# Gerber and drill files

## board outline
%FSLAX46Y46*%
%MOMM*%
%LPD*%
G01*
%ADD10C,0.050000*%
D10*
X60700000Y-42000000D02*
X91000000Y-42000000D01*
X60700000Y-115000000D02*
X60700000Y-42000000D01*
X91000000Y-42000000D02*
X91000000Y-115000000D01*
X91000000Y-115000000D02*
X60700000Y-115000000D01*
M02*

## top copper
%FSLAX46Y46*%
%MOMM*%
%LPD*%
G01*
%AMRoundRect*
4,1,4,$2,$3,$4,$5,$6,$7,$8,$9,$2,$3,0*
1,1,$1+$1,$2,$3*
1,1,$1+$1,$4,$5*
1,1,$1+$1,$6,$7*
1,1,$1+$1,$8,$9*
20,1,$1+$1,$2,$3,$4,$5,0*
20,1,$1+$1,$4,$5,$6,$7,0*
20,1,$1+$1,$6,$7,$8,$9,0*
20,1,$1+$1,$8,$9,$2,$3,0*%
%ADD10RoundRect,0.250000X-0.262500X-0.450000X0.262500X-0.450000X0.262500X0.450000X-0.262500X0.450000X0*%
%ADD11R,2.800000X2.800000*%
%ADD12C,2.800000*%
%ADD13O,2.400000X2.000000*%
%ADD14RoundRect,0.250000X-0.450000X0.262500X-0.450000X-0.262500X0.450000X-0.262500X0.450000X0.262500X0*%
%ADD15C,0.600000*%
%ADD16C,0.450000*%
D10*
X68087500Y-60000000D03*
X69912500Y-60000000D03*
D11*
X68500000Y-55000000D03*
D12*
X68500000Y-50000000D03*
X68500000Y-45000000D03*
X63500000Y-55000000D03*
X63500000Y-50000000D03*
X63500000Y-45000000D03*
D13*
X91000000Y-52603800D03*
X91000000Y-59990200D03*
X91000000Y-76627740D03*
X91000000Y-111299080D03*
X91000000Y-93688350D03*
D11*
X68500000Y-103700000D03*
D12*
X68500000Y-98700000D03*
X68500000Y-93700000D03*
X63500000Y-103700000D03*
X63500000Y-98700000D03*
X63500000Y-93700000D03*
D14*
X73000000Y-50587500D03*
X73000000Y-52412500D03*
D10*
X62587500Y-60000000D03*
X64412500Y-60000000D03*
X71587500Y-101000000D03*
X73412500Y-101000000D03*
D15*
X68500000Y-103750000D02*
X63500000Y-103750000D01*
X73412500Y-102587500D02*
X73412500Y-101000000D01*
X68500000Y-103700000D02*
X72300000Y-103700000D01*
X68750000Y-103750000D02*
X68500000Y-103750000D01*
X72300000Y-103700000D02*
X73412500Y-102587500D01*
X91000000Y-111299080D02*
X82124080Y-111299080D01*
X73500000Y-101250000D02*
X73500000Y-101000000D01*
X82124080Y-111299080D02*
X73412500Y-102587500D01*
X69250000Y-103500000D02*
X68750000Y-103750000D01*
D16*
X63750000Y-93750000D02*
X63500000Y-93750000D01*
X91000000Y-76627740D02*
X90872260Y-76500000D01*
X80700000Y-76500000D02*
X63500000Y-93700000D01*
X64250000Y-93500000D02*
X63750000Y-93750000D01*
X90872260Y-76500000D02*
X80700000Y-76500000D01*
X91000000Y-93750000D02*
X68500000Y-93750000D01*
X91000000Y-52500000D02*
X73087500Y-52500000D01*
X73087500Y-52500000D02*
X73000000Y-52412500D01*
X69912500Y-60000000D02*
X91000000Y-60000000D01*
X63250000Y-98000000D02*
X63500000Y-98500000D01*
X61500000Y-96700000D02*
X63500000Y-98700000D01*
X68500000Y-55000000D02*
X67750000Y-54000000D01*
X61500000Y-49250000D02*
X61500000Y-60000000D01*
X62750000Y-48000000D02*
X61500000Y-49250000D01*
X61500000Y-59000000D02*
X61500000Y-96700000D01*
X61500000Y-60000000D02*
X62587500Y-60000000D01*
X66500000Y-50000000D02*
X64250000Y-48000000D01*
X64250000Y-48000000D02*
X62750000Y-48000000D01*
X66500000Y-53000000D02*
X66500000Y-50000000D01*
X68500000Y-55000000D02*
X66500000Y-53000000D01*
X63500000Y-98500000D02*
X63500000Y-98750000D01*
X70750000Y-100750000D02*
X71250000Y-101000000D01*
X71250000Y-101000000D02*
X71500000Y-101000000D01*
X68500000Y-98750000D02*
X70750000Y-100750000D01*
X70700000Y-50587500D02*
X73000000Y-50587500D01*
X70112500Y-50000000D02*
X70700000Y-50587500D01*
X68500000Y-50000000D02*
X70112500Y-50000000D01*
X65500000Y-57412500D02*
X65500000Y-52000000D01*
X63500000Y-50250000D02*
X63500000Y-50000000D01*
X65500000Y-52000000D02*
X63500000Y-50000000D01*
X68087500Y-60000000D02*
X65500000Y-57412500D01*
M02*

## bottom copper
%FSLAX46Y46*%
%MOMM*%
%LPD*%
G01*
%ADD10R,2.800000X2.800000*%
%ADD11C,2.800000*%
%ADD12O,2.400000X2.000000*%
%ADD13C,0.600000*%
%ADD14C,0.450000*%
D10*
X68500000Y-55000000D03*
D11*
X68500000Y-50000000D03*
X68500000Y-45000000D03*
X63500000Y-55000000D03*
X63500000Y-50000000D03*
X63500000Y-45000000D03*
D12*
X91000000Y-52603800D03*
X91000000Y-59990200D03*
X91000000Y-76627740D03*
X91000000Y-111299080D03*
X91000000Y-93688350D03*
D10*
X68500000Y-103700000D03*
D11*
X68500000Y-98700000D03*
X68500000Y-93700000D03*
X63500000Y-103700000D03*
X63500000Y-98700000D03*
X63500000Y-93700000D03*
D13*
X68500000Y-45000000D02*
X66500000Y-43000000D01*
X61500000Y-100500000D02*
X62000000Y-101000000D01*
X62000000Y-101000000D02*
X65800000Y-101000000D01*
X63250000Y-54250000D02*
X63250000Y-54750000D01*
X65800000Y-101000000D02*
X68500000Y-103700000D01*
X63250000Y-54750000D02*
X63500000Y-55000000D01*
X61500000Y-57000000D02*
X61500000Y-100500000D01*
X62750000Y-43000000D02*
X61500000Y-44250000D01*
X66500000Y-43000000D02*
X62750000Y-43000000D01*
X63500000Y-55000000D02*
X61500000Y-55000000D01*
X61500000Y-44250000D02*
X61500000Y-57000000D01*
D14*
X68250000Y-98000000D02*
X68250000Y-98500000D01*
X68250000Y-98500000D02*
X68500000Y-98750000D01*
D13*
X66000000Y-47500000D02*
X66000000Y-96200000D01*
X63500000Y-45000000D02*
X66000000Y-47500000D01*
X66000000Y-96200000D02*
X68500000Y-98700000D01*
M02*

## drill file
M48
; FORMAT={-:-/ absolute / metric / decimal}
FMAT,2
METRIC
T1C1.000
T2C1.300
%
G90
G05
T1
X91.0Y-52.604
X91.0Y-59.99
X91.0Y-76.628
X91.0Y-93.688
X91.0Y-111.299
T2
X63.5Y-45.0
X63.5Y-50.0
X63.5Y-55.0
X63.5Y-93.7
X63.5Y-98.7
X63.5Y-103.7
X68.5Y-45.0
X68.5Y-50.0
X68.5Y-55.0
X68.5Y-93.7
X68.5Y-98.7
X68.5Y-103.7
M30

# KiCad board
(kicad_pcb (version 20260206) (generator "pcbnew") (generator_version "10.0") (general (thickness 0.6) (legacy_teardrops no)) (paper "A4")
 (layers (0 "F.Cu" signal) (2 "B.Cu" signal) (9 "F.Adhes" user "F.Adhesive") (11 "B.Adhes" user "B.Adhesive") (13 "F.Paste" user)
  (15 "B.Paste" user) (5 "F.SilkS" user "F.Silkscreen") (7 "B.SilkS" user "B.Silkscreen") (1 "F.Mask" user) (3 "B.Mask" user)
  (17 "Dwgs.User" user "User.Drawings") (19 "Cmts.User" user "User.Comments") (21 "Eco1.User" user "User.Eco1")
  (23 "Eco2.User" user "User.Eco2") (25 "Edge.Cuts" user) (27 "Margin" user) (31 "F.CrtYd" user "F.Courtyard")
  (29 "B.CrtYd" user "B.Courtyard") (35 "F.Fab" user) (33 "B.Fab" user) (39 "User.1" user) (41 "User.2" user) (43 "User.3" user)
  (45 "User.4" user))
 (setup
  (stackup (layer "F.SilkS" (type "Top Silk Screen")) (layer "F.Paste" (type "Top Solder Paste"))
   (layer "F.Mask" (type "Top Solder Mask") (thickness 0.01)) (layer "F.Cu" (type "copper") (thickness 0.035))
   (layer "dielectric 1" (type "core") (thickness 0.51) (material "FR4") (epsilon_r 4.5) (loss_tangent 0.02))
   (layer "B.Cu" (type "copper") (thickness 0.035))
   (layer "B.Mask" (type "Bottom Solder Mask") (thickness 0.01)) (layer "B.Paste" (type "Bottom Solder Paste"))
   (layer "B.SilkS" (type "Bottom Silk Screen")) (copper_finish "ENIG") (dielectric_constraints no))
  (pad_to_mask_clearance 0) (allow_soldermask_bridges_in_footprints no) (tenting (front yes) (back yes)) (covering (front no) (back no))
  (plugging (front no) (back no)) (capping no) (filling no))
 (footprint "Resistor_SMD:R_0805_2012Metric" (layer "F.Cu") (at 69 60)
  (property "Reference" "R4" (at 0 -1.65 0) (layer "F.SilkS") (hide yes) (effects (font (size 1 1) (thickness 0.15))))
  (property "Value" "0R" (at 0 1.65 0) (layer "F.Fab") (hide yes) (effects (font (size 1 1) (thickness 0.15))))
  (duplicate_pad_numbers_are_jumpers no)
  (pad "1" smd roundrect (at -0.9125 0) (size 1.025 1.4) (layers "F.Cu" "F.Mask" "F.Paste") (roundrect_rratio 0.243902) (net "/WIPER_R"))
  (pad "2" smd roundrect (at 0.9125 0) (size 1.025 1.4) (layers "F.Cu" "F.Mask" "F.Paste") (roundrect_rratio 0.243902) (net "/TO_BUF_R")))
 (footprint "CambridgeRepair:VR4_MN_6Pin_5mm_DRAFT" (layer "F.Cu") (at 63.5 50)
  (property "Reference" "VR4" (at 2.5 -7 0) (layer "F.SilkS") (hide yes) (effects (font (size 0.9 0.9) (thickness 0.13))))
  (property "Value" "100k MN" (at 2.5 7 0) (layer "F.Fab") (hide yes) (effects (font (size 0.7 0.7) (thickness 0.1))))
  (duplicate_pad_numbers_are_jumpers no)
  (pad "1" thru_hole rect (at 5 5) (size 2.8 2.8) (drill 1.3) (layers "*.Cu" "*.Mask") (remove_unused_layers no) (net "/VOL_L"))
  (pad "2" thru_hole circle (at 5 0) (size 2.8 2.8) (drill 1.3) (layers "*.Cu" "*.Mask") (remove_unused_layers no) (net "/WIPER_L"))
  (pad "3" thru_hole circle (at 5 -5) (size 2.8 2.8) (drill 1.3) (layers "*.Cu" "*.Mask") (remove_unused_layers no) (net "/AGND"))
  (pad "4" thru_hole circle (at 0 5) (size 2.8 2.8) (drill 1.3) (layers "*.Cu" "*.Mask") (remove_unused_layers no) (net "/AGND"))
  (pad "5" thru_hole circle (at 0 0) (size 2.8 2.8) (drill 1.3) (layers "*.Cu" "*.Mask") (remove_unused_layers no) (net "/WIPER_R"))
  (pad "6" thru_hole circle (at 0 -5) (size 2.8 2.8) (drill 1.3) (layers "*.Cu" "*.Mask") (remove_unused_layers no) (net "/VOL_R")))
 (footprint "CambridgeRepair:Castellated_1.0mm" (layer "F.Cu") (at 91 52.6038)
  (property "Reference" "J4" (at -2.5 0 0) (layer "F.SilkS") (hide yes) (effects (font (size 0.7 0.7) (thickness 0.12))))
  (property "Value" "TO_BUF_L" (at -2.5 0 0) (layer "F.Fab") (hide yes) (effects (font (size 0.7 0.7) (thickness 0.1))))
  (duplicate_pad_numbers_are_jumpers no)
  (pad "1" thru_hole oval (at 0 0) (size 2.4 2) (drill 1) (layers "*.Cu" "*.Mask") (remove_unused_layers no) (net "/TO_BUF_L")
   (solder_mask_margin 0.05)))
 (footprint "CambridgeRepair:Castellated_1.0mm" (layer "F.Cu") (at 91 59.9902)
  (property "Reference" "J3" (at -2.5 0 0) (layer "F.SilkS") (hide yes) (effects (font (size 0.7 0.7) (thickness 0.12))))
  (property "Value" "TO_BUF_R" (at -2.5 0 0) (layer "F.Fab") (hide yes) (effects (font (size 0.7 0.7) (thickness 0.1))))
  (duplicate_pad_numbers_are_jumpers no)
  (pad "1" thru_hole oval (at 0 0) (size 2.4 2) (drill 1) (layers "*.Cu" "*.Mask") (remove_unused_layers no) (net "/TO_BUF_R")
   (solder_mask_margin 0.05)))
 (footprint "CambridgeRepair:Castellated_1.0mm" (layer "F.Cu") (at 91 76.62774)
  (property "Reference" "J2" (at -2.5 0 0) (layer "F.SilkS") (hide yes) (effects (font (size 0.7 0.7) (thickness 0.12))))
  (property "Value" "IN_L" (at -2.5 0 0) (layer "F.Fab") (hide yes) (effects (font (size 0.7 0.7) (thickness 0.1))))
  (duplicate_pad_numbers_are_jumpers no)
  (pad "1" thru_hole oval (at 0 0) (size 2.4 2) (drill 1) (layers "*.Cu" "*.Mask") (remove_unused_layers no) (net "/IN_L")
   (solder_mask_margin 0.05)))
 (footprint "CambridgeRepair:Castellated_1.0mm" (layer "F.Cu") (at 91 111.29908)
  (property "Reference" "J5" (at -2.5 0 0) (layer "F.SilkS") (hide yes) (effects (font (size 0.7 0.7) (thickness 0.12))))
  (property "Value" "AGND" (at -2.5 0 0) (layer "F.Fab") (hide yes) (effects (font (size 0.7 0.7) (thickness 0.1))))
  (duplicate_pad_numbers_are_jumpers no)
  (pad "1" thru_hole oval (at 0 0) (size 2.4 2) (drill 1) (layers "*.Cu" "*.Mask") (remove_unused_layers no) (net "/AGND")
   (solder_mask_margin 0.05)))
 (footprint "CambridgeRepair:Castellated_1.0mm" (layer "F.Cu") (at 91 93.68835)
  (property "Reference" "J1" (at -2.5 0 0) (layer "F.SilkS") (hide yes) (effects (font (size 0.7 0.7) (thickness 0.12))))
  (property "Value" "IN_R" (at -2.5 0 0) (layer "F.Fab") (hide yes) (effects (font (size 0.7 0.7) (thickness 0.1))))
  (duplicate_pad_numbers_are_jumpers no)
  (pad "1" thru_hole oval (at 0 0) (size 2.4 2) (drill 1) (layers "*.Cu" "*.Mask") (remove_unused_layers no) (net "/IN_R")
   (solder_mask_margin 0.05)))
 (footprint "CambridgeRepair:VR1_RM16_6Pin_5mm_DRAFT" (layer "F.Cu") (at 63.5 98.7)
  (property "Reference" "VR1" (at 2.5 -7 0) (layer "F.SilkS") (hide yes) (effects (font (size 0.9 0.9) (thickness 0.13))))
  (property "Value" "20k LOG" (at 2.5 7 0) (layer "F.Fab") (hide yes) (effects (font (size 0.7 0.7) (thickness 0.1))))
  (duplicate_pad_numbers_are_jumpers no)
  (pad "1" thru_hole rect (at 5 5) (size 2.8 2.8) (drill 1.3) (layers "*.Cu" "*.Mask") (remove_unused_layers no) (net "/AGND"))
  (pad "2" thru_hole circle (at 5 0) (size 2.8 2.8) (drill 1.3) (layers "*.Cu" "*.Mask") (remove_unused_layers no) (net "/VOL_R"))
  (pad "3" thru_hole circle (at 5 -5) (size 2.8 2.8) (drill 1.3) (layers "*.Cu" "*.Mask") (remove_unused_layers no) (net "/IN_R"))
  (pad "4" thru_hole circle (at 0 5) (size 2.8 2.8) (drill 1.3) (layers "*.Cu" "*.Mask") (remove_unused_layers no) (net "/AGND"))
  (pad "5" thru_hole circle (at 0 0) (size 2.8 2.8) (drill 1.3) (layers "*.Cu" "*.Mask") (remove_unused_layers no) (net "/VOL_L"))
  (pad "6" thru_hole circle (at 0 -5) (size 2.8 2.8) (drill 1.3) (layers "*.Cu" "*.Mask") (remove_unused_layers no) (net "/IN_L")))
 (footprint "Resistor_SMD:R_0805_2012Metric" (layer "F.Cu") (at 73 51.5 -90)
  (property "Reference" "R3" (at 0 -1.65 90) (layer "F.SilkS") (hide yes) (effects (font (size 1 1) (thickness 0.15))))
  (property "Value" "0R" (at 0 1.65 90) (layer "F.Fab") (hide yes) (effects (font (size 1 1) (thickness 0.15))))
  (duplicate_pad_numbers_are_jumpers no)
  (pad "1" smd roundrect (at -0.9125 0 270) (size 1.025 1.4) (layers "F.Cu" "F.Mask" "F.Paste") (roundrect_rratio 0.243902) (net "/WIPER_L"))
  (pad "2" smd roundrect (at 0.9125 0 270) (size 1.025 1.4) (layers "F.Cu" "F.Mask" "F.Paste") (roundrect_rratio 0.243902) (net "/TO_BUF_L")))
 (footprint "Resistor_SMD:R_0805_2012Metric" (layer "F.Cu") (at 63.5 60)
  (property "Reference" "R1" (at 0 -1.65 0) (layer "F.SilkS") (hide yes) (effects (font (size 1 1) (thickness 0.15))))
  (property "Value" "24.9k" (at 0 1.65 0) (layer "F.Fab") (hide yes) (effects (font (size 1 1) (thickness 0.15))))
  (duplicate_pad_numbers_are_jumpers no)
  (pad "1" smd roundrect (at -0.9125 0) (size 1.025 1.4) (layers "F.Cu" "F.Mask" "F.Paste") (roundrect_rratio 0.243902) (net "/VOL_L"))
  (pad "2" smd roundrect (at 0.9125 0) (size 1.025 1.4) (layers "F.Cu" "F.Mask" "F.Paste") (roundrect_rratio 0.243902) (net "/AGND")))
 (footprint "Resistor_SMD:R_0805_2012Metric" (layer "F.Cu") (at 72.5 101)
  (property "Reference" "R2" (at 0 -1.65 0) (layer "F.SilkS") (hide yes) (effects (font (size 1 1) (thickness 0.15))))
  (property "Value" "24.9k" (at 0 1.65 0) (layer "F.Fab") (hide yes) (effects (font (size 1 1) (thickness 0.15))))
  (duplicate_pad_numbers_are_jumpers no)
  (pad "1" smd roundrect (at -0.9125 0) (size 1.025 1.4) (layers "F.Cu" "F.Mask" "F.Paste") (roundrect_rratio 0.243902) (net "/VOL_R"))
  (pad "2" smd roundrect (at 0.9125 0) (size 1.025 1.4) (layers "F.Cu" "F.Mask" "F.Paste") (roundrect_rratio 0.243902) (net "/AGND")))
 (gr_line (start 60.7 42) (end 91 42) (stroke (width 0.05) (type default)) (layer "Edge.Cuts"))
 (gr_line (start 60.7 115) (end 60.7 42) (stroke (width 0.05) (type default)) (layer "Edge.Cuts"))
 (gr_line (start 91 42) (end 91 115) (stroke (width 0.05) (type default)) (layer "Edge.Cuts"))
 (gr_line (start 91 115) (end 60.7 115) (stroke (width 0.05) (type default)) (layer "Edge.Cuts"))
 (segment (start 68.5 103.75) (end 63.5 103.75) (width 0.6) (layer "F.Cu") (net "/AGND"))
 (segment (start 73.4125 102.5875) (end 73.4125 101) (width 0.6) (layer "F.Cu") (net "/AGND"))
 (segment (start 68.5 103.7) (end 72.3 103.7) (width 0.6) (layer "F.Cu") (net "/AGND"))
 (segment (start 68.75 103.75) (end 68.5 103.75) (width 0.6) (layer "F.Cu") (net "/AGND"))
 (segment (start 72.3 103.7) (end 73.4125 102.5875) (width 0.6) (layer "F.Cu") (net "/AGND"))
 (segment (start 91 111.29908) (end 82.12408 111.29908) (width 0.6) (layer "F.Cu") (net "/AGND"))
 (segment (start 73.5 101.25) (end 73.5 101) (width 0.6) (layer "F.Cu") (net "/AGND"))
 (segment (start 82.12408 111.29908) (end 73.4125 102.5875) (width 0.6) (layer "F.Cu") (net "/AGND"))
 (segment (start 69.25 103.5) (end 68.75 103.75) (width 0.6) (layer "F.Cu") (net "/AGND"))
 (segment (start 68.5 45) (end 66.5 43) (width 0.6) (layer "B.Cu") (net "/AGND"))
 (segment (start 61.5 100.5) (end 62 101) (width 0.6) (layer "B.Cu") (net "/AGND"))
 (segment (start 62 101) (end 65.8 101) (width 0.6) (layer "B.Cu") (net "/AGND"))
 (segment (start 63.25 54.25) (end 63.25 54.75) (width 0.6) (layer "B.Cu") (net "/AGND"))
 (segment (start 65.8 101) (end 68.5 103.7) (width 0.6) (layer "B.Cu") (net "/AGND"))
 (segment (start 63.25 54.75) (end 63.5 55) (width 0.6) (layer "B.Cu") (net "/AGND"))
 (segment (start 61.5 57) (end 61.5 100.5) (width 0.6) (layer "B.Cu") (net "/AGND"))
 (segment (start 62.75 43) (end 61.5 44.25) (width 0.6) (layer "B.Cu") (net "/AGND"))
 (segment (start 66.5 43) (end 62.75 43) (width 0.6) (layer "B.Cu") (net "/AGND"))
 (segment (start 63.5 55) (end 61.5 55) (width 0.6) (layer "B.Cu") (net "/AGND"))
 (segment (start 61.5 44.25) (end 61.5 57) (width 0.6) (layer "B.Cu") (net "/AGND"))
 (segment (start 63.75 93.75) (end 63.5 93.75) (width 0.45) (layer "F.Cu") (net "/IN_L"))
 (segment (start 91 76.62774) (end 90.87226 76.5) (width 0.45) (layer "F.Cu") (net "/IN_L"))
 (segment (start 80.7 76.5) (end 63.5 93.7) (width 0.45) (layer "F.Cu") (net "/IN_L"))
 (segment (start 64.25 93.5) (end 63.75 93.75) (width 0.45) (layer "F.Cu") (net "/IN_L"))
 (segment (start 90.87226 76.5) (end 80.7 76.5) (width 0.45) (layer "F.Cu") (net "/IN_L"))
 (segment (start 91 93.75) (end 68.5 93.75) (width 0.45) (layer "F.Cu") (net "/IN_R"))
 (segment (start 91 52.5) (end 73.0875 52.5) (width 0.45) (layer "F.Cu") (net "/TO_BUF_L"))
 (segment (start 73.0875 52.5) (end 73 52.4125) (width 0.45) (layer "F.Cu") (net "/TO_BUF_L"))
 (segment (start 69.9125 60) (end 91 60) (width 0.45) (layer "F.Cu") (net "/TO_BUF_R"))
 (segment (start 63.25 98) (end 63.5 98.5) (width 0.45) (layer "F.Cu") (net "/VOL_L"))
 (segment (start 61.5 96.7) (end 63.5 98.7) (width 0.45) (layer "F.Cu") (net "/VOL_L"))
 (segment (start 68.5 55) (end 67.75 54) (width 0.45) (layer "F.Cu") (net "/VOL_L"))
 (segment (start 61.5 49.25) (end 61.5 60) (width 0.45) (layer "F.Cu") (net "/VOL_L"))
 (segment (start 62.75 48) (end 61.5 49.25) (width 0.45) (layer "F.Cu") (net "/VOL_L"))
 (segment (start 61.5 59) (end 61.5 96.7) (width 0.45) (layer "F.Cu") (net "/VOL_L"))
 (segment (start 61.5 60) (end 62.5875 60) (width 0.45) (layer "F.Cu") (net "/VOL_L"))
 (segment (start 66.5 50) (end 64.25 48) (width 0.45) (layer "F.Cu") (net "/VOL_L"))
 (segment (start 64.25 48) (end 62.75 48) (width 0.45) (layer "F.Cu") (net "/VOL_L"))
 (segment (start 66.5 53) (end 66.5 50) (width 0.45) (layer "F.Cu") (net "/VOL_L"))
 (segment (start 68.5 55) (end 66.5 53) (width 0.45) (layer "F.Cu") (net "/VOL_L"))
 (segment (start 63.5 98.5) (end 63.5 98.75) (width 0.45) (layer "F.Cu") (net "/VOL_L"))
 (segment (start 70.75 100.75) (end 71.25 101) (width 0.45) (layer "F.Cu") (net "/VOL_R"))
 (segment (start 71.25 101) (end 71.5 101) (width 0.45) (layer "F.Cu") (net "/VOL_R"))
 (segment (start 68.5 98.75) (end 70.75 100.75) (width 0.45) (layer "F.Cu") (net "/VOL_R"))
 (segment (start 68.25 98) (end 68.25 98.5) (width 0.45) (layer "B.Cu") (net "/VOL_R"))
 (segment (start 68.25 98.5) (end 68.5 98.75) (width 0.45) (layer "B.Cu") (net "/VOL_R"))
 (segment (start 66 47.5) (end 66 96.2) (width 0.6) (layer "B.Cu") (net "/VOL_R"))
 (segment (start 63.5 45) (end 66 47.5) (width 0.6) (layer "B.Cu") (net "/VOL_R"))
 (segment (start 66 96.2) (end 68.5 98.7) (width 0.6) (layer "B.Cu") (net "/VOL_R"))
 (segment (start 70.7 50.5875) (end 73 50.5875) (width 0.45) (layer "F.Cu") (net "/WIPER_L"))
 (segment (start 70.1125 50) (end 70.7 50.5875) (width 0.45) (layer "F.Cu") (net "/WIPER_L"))
 (segment (start 68.5 50) (end 70.1125 50) (width 0.45) (layer "F.Cu") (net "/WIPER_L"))
 (segment (start 65.5 57.4125) (end 65.5 52) (width 0.45) (layer "F.Cu") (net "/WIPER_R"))
 (segment (start 63.5 50.25) (end 63.5 50) (width 0.45) (layer "F.Cu") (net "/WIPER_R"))
 (segment (start 65.5 52) (end 63.5 50) (width 0.45) (layer "F.Cu") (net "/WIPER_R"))
 (segment (start 68.0875 60) (end 65.5 57.4125) (width 0.45) (layer "F.Cu") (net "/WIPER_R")))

